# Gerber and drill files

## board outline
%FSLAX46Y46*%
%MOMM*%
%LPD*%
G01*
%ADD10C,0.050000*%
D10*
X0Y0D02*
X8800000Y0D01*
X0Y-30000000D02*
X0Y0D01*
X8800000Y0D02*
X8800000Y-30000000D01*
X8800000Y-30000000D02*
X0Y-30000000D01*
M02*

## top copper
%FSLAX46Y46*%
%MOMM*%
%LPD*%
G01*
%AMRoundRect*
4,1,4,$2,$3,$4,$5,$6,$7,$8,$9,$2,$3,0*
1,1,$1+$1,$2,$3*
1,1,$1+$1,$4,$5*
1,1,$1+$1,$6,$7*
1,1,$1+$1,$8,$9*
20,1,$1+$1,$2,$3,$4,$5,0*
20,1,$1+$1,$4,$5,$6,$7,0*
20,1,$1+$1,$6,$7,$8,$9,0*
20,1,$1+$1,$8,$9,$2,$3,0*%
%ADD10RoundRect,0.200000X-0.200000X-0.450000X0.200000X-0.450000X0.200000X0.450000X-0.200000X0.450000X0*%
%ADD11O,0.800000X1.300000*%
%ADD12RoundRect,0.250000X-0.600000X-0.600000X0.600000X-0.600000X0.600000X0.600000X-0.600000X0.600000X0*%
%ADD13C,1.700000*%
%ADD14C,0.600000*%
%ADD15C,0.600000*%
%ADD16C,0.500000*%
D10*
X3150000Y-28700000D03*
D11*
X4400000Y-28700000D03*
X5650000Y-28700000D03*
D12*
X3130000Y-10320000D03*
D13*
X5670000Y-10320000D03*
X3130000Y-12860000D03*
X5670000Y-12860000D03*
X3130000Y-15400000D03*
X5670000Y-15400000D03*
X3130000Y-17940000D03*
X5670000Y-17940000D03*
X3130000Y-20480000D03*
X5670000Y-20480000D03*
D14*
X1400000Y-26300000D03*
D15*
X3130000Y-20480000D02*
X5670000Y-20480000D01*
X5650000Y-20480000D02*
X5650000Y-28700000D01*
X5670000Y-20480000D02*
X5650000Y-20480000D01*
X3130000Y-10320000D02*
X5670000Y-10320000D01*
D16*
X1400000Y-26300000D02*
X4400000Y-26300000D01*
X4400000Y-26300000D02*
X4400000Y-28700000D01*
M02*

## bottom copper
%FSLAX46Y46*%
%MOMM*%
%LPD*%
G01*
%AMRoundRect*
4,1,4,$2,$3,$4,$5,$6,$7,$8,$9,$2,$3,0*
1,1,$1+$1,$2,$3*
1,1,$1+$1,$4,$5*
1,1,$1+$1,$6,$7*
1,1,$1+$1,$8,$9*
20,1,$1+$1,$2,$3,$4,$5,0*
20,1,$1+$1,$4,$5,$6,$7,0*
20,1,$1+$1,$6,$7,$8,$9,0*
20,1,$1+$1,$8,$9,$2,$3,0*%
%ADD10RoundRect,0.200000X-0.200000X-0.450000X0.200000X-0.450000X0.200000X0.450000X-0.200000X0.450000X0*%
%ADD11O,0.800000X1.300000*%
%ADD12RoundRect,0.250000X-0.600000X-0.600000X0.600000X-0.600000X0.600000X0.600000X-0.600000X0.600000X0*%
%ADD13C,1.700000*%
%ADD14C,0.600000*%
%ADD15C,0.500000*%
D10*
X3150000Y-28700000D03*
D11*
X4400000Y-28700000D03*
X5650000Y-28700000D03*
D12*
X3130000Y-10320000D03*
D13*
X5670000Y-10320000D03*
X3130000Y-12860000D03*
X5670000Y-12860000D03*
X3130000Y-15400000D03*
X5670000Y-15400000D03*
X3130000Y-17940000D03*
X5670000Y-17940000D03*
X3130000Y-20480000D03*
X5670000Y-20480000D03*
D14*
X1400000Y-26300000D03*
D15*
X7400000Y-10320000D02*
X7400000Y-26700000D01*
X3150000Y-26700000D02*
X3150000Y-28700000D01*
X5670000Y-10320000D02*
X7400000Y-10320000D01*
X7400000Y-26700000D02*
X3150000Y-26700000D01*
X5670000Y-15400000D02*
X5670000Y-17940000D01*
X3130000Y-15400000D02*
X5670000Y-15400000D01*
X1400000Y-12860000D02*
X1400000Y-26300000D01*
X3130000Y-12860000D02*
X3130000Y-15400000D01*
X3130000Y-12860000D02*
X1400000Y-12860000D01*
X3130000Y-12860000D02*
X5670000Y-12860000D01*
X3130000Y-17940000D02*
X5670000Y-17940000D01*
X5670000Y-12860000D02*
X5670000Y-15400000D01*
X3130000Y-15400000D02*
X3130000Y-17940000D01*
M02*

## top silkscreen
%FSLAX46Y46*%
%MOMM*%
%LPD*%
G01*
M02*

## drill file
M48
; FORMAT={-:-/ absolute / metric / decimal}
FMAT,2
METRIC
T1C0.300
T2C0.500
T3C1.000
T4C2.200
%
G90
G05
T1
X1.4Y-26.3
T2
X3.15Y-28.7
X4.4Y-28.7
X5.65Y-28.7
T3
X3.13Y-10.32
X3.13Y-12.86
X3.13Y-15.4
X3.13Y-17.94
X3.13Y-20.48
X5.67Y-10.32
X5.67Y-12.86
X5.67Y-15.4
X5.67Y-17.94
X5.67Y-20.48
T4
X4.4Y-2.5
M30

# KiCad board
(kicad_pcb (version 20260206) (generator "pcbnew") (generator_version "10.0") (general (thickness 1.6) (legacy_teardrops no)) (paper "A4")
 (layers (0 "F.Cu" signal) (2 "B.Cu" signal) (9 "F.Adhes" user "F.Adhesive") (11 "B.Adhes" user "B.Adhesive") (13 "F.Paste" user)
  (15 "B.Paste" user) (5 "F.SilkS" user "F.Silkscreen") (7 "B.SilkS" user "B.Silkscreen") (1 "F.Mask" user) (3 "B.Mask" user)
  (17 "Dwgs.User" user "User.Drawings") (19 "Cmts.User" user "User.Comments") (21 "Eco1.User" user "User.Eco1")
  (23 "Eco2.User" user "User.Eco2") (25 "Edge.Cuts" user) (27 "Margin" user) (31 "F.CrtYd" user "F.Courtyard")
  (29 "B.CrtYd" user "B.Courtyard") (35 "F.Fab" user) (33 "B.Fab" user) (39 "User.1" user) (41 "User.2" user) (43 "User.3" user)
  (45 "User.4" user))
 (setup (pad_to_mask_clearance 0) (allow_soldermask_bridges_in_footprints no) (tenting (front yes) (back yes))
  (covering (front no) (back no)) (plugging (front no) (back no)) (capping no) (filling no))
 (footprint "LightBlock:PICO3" (layer "F.Cu") (at 3.15 28.7)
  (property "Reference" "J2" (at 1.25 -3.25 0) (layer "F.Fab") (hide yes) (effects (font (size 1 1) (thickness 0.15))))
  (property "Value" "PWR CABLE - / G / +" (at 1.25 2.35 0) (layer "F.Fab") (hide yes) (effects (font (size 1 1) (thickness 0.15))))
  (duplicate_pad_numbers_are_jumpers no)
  (pad "1" thru_hole roundrect (at 0 0) (size 0.8 1.3) (drill 0.5) (layers "*.Cu" "*.Mask") (remove_unused_layers no)
   (roundrect_rratio 0.25) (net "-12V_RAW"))
  (pad "2" thru_hole oval (at 1.25 0) (size 0.8 1.3) (drill 0.5) (layers "*.Cu" "*.Mask") (remove_unused_layers no) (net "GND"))
  (pad "3" thru_hole oval (at 2.5 0) (size 0.8 1.3) (drill 0.5) (layers "*.Cu" "*.Mask") (remove_unused_layers no) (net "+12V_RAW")))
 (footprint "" (layer "F.Cu") (at 4.4 2.5)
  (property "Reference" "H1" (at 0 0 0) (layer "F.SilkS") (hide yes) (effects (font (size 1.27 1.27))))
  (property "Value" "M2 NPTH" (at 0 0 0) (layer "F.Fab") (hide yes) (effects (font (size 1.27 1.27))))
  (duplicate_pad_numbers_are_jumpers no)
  (pad "" np_thru_hole circle (at 0 0) (size 2.2 2.2) (drill 2.2) (layers "*.Cu" "*.Mask")))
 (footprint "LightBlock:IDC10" (layer "F.Cu") (at 3.13 10.32)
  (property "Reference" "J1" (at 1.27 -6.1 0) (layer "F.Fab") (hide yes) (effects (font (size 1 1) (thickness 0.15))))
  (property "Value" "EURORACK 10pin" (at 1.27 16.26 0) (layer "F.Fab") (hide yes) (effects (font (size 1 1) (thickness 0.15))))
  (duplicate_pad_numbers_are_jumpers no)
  (pad "1" thru_hole roundrect (at 0 0) (size 1.7 1.7) (drill 1) (layers "*.Cu" "*.Mask") (remove_unused_layers no)
   (roundrect_rratio 0.147059) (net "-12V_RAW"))
  (pad "2" thru_hole circle (at 2.54 0) (size 1.7 1.7) (drill 1) (layers "*.Cu" "*.Mask") (remove_unused_layers no) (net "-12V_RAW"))
  (pad "3" thru_hole circle (at 0 2.54) (size 1.7 1.7) (drill 1) (layers "*.Cu" "*.Mask") (remove_unused_layers no) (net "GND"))
  (pad "4" thru_hole circle (at 2.54 2.54) (size 1.7 1.7) (drill 1) (layers "*.Cu" "*.Mask") (remove_unused_layers no) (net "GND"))
  (pad "5" thru_hole circle (at 0 5.08) (size 1.7 1.7) (drill 1) (layers "*.Cu" "*.Mask") (remove_unused_layers no) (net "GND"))
  (pad "6" thru_hole circle (at 2.54 5.08) (size 1.7 1.7) (drill 1) (layers "*.Cu" "*.Mask") (remove_unused_layers no) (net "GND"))
  (pad "7" thru_hole circle (at 0 7.62) (size 1.7 1.7) (drill 1) (layers "*.Cu" "*.Mask") (remove_unused_layers no) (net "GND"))
  (pad "8" thru_hole circle (at 2.54 7.62) (size 1.7 1.7) (drill 1) (layers "*.Cu" "*.Mask") (remove_unused_layers no) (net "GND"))
  (pad "9" thru_hole circle (at 0 10.16) (size 1.7 1.7) (drill 1) (layers "*.Cu" "*.Mask") (remove_unused_layers no) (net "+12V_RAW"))
  (pad "10" thru_hole circle (at 2.54 10.16) (size 1.7 1.7) (drill 1) (layers "*.Cu" "*.Mask") (remove_unused_layers no) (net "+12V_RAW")))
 (gr_line (start 0 0) (end 8.8 0) (stroke (width 0.05) (type default)) (layer "Edge.Cuts"))
 (gr_line (start 0 30) (end 0 0) (stroke (width 0.05) (type default)) (layer "Edge.Cuts"))
 (gr_line (start 8.8 0) (end 8.8 30) (stroke (width 0.05) (type default)) (layer "Edge.Cuts"))
 (gr_line (start 8.8 30) (end 0 30) (stroke (width 0.05) (type default)) (layer "Edge.Cuts"))
 (segment (start 3.13 20.48) (end 5.67 20.48) (width 0.6) (layer "F.Cu") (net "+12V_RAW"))
 (segment (start 5.65 20.48) (end 5.65 28.7) (width 0.6) (layer "F.Cu") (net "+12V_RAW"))
 (segment (start 5.67 20.48) (end 5.65 20.48) (width 0.6) (layer "F.Cu") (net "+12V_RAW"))
 (segment (start 3.13 10.32) (end 5.67 10.32) (width 0.6) (layer "F.Cu") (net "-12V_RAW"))
 (segment (start 7.4 10.32) (end 7.4 26.7) (width 0.5) (layer "B.Cu") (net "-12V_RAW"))
 (segment (start 3.15 26.7) (end 3.15 28.7) (width 0.5) (layer "B.Cu") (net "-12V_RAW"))
 (segment (start 5.67 10.32) (end 7.4 10.32) (width 0.5) (layer "B.Cu") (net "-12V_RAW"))
 (segment (start 7.4 26.7) (end 3.15 26.7) (width 0.5) (layer "B.Cu") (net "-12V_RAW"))
 (segment (start 1.4 26.3) (end 4.4 26.3) (width 0.5) (layer "F.Cu") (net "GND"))
 (segment (start 4.4 26.3) (end 4.4 28.7) (width 0.5) (layer "F.Cu") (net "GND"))
 (via (at 1.4 26.3) (size 0.6) (drill 0.3) (layers "F.Cu" "B.Cu") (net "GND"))
 (segment (start 5.67 15.4) (end 5.67 17.94) (width 0.5) (layer "B.Cu") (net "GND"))
 (segment (start 3.13 15.4) (end 5.67 15.4) (width 0.5) (layer "B.Cu") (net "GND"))
 (segment (start 1.4 12.86) (end 1.4 26.3) (width 0.5) (layer "B.Cu") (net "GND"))
 (segment (start 3.13 12.86) (end 3.13 15.4) (width 0.5) (layer "B.Cu") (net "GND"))
 (segment (start 3.13 12.86) (end 1.4 12.86) (width 0.5) (layer "B.Cu") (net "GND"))
 (segment (start 3.13 12.86) (end 5.67 12.86) (width 0.5) (layer "B.Cu") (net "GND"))
 (segment (start 3.13 17.94) (end 5.67 17.94) (width 0.5) (layer "B.Cu") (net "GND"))
 (segment (start 5.67 12.86) (end 5.67 15.4) (width 0.5) (layer "B.Cu") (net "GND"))
 (segment (start 3.13 15.4) (end 3.13 17.94) (width 0.5) (layer "B.Cu") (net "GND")))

